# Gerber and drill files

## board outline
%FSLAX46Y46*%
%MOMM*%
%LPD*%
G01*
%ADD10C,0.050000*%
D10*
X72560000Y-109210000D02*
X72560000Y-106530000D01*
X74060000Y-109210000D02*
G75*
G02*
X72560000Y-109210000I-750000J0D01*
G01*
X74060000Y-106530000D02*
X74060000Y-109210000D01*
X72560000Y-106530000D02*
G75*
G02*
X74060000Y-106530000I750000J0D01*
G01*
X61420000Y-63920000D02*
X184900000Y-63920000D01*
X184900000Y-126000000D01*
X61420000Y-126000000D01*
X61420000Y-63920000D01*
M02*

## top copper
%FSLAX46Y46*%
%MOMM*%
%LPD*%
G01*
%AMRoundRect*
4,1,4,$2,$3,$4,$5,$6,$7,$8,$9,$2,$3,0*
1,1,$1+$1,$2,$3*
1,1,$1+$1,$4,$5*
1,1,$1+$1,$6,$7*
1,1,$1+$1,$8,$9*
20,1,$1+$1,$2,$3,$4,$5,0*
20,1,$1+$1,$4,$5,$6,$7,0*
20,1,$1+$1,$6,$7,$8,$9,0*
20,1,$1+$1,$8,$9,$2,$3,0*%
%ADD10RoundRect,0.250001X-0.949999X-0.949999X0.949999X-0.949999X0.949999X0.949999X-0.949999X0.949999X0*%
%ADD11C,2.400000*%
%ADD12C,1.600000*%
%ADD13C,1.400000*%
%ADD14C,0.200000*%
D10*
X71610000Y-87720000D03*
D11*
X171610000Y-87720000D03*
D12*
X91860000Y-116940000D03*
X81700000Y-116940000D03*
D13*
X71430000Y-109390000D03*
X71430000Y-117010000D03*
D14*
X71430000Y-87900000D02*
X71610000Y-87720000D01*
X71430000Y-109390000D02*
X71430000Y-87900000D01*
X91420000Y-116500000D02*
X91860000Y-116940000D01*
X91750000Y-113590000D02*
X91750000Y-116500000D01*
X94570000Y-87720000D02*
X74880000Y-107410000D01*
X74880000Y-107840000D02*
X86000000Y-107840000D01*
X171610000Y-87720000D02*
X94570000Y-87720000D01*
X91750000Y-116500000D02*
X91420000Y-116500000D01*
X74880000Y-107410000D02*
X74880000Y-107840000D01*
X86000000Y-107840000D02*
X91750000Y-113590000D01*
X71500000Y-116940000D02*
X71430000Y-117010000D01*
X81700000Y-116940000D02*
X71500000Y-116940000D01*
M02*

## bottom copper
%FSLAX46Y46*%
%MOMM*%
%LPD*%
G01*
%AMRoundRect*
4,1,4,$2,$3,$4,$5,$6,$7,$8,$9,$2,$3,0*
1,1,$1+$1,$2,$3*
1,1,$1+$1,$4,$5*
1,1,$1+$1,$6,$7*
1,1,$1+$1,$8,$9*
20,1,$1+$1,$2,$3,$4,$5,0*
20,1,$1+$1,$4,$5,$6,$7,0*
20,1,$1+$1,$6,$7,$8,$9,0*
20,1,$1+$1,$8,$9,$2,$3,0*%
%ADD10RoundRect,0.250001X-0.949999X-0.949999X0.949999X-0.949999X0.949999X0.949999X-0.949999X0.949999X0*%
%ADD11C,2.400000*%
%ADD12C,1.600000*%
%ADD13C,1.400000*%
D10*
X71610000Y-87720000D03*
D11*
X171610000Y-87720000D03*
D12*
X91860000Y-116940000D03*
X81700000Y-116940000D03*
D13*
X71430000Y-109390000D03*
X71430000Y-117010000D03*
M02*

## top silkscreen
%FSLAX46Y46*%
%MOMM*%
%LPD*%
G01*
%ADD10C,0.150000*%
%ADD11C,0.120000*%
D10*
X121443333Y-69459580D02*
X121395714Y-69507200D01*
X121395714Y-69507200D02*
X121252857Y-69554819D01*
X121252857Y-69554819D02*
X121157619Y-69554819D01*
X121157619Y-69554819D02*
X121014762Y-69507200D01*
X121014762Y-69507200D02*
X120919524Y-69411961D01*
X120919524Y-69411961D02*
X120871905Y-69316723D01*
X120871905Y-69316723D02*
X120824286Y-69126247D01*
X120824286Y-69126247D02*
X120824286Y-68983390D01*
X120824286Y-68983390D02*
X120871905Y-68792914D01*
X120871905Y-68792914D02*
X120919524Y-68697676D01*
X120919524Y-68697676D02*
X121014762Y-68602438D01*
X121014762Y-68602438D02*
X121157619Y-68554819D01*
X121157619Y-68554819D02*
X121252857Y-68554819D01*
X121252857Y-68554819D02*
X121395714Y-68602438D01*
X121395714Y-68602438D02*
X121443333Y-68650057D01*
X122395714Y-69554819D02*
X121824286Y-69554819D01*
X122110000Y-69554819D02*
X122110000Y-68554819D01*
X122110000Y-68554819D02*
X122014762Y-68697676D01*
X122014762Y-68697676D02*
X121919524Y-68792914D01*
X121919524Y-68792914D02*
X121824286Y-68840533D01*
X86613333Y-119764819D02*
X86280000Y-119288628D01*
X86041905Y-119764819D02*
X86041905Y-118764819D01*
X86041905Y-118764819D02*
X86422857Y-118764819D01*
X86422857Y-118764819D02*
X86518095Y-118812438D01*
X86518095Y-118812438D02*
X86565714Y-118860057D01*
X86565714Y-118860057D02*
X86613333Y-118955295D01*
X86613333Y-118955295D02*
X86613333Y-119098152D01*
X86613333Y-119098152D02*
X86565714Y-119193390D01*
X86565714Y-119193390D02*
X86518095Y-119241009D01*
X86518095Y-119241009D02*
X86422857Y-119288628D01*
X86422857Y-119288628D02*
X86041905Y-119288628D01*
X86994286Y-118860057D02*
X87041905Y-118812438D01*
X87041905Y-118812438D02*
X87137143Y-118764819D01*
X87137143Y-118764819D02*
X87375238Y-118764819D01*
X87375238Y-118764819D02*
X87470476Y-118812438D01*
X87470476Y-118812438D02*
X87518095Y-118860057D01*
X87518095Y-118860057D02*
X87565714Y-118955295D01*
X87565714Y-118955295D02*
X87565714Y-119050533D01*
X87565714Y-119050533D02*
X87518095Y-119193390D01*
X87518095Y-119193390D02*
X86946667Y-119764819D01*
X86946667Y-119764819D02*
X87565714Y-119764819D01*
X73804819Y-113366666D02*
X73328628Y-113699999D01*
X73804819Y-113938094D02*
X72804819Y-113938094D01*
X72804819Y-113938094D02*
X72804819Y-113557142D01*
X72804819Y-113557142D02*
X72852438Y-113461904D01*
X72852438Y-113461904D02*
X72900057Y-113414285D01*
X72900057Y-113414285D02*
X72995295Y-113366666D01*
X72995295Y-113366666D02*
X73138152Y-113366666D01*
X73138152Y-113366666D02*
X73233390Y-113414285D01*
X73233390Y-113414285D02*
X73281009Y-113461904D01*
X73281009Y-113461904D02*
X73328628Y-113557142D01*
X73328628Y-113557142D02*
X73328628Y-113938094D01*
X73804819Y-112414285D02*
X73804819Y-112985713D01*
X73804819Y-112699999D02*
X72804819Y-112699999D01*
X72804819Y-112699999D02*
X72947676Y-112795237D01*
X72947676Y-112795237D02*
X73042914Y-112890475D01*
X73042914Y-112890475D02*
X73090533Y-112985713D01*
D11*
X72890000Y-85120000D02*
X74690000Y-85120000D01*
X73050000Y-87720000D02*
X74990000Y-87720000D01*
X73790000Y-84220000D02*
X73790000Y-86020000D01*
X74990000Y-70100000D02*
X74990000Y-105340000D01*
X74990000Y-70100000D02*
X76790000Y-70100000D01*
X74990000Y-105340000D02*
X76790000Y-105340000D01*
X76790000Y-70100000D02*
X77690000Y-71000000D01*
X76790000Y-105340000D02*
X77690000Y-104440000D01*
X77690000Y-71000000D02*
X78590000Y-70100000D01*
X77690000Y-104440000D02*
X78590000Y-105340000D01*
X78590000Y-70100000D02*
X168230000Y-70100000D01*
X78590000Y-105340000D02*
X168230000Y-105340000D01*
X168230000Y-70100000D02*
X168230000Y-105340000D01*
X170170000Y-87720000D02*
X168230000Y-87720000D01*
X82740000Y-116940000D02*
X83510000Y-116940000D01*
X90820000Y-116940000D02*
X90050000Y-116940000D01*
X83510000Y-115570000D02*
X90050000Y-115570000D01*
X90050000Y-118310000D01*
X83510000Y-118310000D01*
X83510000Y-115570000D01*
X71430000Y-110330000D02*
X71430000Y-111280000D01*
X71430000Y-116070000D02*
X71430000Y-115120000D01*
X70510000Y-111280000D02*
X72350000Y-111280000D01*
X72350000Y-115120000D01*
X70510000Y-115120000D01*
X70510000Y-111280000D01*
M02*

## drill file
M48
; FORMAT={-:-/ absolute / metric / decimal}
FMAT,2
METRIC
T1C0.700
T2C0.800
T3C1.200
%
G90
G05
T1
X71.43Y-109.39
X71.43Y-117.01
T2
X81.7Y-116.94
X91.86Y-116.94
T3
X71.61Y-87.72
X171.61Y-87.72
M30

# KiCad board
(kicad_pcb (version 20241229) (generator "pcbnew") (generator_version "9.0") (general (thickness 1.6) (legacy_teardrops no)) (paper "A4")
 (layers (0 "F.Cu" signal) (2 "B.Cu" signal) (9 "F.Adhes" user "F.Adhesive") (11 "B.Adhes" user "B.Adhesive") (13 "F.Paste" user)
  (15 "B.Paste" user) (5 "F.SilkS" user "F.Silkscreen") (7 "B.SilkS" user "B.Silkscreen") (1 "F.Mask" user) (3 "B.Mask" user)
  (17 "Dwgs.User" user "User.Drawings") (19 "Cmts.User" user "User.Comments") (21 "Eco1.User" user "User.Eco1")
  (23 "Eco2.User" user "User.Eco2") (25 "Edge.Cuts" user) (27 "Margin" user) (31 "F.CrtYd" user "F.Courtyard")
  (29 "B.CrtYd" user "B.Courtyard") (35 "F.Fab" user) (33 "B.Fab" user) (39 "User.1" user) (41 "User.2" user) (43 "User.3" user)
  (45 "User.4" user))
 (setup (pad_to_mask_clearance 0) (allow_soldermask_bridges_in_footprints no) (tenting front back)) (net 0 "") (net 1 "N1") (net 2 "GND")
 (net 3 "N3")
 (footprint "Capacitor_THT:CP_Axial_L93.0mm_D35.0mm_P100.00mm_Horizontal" (layer "F.Cu") (at 71.61 87.72)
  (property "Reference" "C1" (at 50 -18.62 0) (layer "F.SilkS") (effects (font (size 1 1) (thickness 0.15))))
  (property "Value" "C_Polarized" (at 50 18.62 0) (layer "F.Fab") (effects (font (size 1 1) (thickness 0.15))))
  (fp_line (start 1.28 -2.6) (end 3.08 -2.6) (stroke (width 0.12) (type solid)) (layer "F.SilkS"))
  (fp_line (start 1.44 0) (end 3.38 0) (stroke (width 0.12) (type solid)) (layer "F.SilkS"))
  (fp_line (start 2.18 -3.5) (end 2.18 -1.7) (stroke (width 0.12) (type solid)) (layer "F.SilkS"))
  (fp_line (start 3.38 -17.62) (end 3.38 17.62) (stroke (width 0.12) (type solid)) (layer "F.SilkS"))
  (fp_line (start 3.38 -17.62) (end 5.18 -17.62) (stroke (width 0.12) (type solid)) (layer "F.SilkS"))
  (fp_line (start 3.38 17.62) (end 5.18 17.62) (stroke (width 0.12) (type solid)) (layer "F.SilkS"))
  (fp_line (start 5.18 -17.62) (end 6.08 -16.72) (stroke (width 0.12) (type solid)) (layer "F.SilkS"))
  (fp_line (start 5.18 17.62) (end 6.08 16.72) (stroke (width 0.12) (type solid)) (layer "F.SilkS"))
  (fp_line (start 6.08 -16.72) (end 6.98 -17.62) (stroke (width 0.12) (type solid)) (layer "F.SilkS"))
  (fp_line (start 6.08 16.72) (end 6.98 17.62) (stroke (width 0.12) (type solid)) (layer "F.SilkS"))
  (fp_line (start 6.98 -17.62) (end 96.62 -17.62) (stroke (width 0.12) (type solid)) (layer "F.SilkS"))
  (fp_line (start 6.98 17.62) (end 96.62 17.62) (stroke (width 0.12) (type solid)) (layer "F.SilkS"))
  (fp_line (start 96.62 -17.62) (end 96.62 17.62) (stroke (width 0.12) (type solid)) (layer "F.SilkS"))
  (fp_line (start 98.56 0) (end 96.62 0) (stroke (width 0.12) (type solid)) (layer "F.SilkS"))
  (pad "1" thru_hole roundrect (at 0 0) (size 2.4 2.4) (drill 1.2) (layers "*.Cu" "*.Mask") (remove_unused_layers no)
   (roundrect_rratio 0.104167) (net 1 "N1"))
  (pad "2" thru_hole circle (at 100 0) (size 2.4 2.4) (drill 1.2) (layers "*.Cu" "*.Mask") (remove_unused_layers no) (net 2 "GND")))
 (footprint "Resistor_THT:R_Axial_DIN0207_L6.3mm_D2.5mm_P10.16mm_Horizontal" (layer "F.Cu") (at 91.86 116.94 180)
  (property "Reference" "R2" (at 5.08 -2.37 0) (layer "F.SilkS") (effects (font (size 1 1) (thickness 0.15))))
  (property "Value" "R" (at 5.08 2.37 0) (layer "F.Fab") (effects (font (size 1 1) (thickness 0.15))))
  (fp_line (start 9.12 0) (end 8.35 0) (stroke (width 0.12) (type solid)) (layer "F.SilkS"))
  (fp_line (start 1.04 0) (end 1.81 0) (stroke (width 0.12) (type solid)) (layer "F.SilkS"))
  (fp_rect (start 1.81 -1.37) (end 8.35 1.37) (stroke (width 0.12) (type solid)) (fill no) (layer "F.SilkS"))
  (pad "1" thru_hole circle (at 0 0 180) (size 1.6 1.6) (drill 0.8) (layers "*.Cu" "*.Mask") (remove_unused_layers no) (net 2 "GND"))
  (pad "2" thru_hole circle (at 10.16 0 180) (size 1.6 1.6) (drill 0.8) (layers "*.Cu" "*.Mask") (remove_unused_layers no) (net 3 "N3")))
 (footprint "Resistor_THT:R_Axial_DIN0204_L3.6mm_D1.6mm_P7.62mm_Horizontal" (layer "F.Cu") (at 71.43 109.39 -90)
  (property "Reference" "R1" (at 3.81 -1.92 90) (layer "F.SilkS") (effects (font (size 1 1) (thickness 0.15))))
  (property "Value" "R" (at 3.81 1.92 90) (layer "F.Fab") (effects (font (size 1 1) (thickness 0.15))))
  (fp_line (start 0.94 0) (end 1.89 0) (stroke (width 0.12) (type solid)) (layer "F.SilkS"))
  (fp_line (start 6.68 0) (end 5.73 0) (stroke (width 0.12) (type solid)) (layer "F.SilkS"))
  (fp_rect (start 1.89 -0.92) (end 5.73 0.92) (stroke (width 0.12) (type solid)) (fill no) (layer "F.SilkS"))
  (pad "1" thru_hole circle (at 0 0 270) (size 1.4 1.4) (drill 0.7) (layers "*.Cu" "*.Mask") (remove_unused_layers no) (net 1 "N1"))
  (pad "2" thru_hole circle (at 7.62 0 270) (size 1.4 1.4) (drill 0.7) (layers "*.Cu" "*.Mask") (remove_unused_layers no) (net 3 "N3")))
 (gr_line (start 72.56 109.21) (end 72.56 106.53) (stroke (width 0.05) (type default)) (layer "Edge.Cuts"))
 (gr_arc (start 74.06 109.21) (mid 73.31 109.96) (end 72.56 109.21) (stroke (width 0.05) (type default)) (layer "Edge.Cuts"))
 (gr_line (start 74.06 106.53) (end 74.06 109.21) (stroke (width 0.05) (type default)) (layer "Edge.Cuts"))
 (gr_arc (start 72.56 106.53) (mid 73.31 105.78) (end 74.06 106.53) (stroke (width 0.05) (type default)) (layer "Edge.Cuts"))
 (gr_rect (start 61.42 63.92) (end 184.9 126) (stroke (width 0.05) (type default)) (fill no) (layer "Edge.Cuts"))
 (segment (start 71.43 87.9) (end 71.61 87.72) (width 0.2) (layer "F.Cu") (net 1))
 (segment (start 71.43 109.39) (end 71.43 87.9) (width 0.2) (layer "F.Cu") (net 1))
 (segment (start 91.42 116.5) (end 91.86 116.94) (width 0.2) (layer "F.Cu") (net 2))
 (segment (start 91.75 113.59) (end 91.75 116.5) (width 0.2) (layer "F.Cu") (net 2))
 (segment (start 94.57 87.72) (end 74.88 107.41) (width 0.2) (layer "F.Cu") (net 2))
 (segment (start 74.88 107.84) (end 86 107.84) (width 0.2) (layer "F.Cu") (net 2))
 (segment (start 171.61 87.72) (end 94.57 87.72) (width 0.2) (layer "F.Cu") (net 2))
 (segment (start 91.75 116.5) (end 91.42 116.5) (width 0.2) (layer "F.Cu") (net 2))
 (segment (start 74.88 107.41) (end 74.88 107.84) (width 0.2) (layer "F.Cu") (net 2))
 (segment (start 86 107.84) (end 91.75 113.59) (width 0.2) (layer "F.Cu") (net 2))
 (segment (start 71.5 116.94) (end 71.43 117.01) (width 0.2) (layer "F.Cu") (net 3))
 (segment (start 81.7 116.94) (end 71.5 116.94) (width 0.2) (layer "F.Cu") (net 3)))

